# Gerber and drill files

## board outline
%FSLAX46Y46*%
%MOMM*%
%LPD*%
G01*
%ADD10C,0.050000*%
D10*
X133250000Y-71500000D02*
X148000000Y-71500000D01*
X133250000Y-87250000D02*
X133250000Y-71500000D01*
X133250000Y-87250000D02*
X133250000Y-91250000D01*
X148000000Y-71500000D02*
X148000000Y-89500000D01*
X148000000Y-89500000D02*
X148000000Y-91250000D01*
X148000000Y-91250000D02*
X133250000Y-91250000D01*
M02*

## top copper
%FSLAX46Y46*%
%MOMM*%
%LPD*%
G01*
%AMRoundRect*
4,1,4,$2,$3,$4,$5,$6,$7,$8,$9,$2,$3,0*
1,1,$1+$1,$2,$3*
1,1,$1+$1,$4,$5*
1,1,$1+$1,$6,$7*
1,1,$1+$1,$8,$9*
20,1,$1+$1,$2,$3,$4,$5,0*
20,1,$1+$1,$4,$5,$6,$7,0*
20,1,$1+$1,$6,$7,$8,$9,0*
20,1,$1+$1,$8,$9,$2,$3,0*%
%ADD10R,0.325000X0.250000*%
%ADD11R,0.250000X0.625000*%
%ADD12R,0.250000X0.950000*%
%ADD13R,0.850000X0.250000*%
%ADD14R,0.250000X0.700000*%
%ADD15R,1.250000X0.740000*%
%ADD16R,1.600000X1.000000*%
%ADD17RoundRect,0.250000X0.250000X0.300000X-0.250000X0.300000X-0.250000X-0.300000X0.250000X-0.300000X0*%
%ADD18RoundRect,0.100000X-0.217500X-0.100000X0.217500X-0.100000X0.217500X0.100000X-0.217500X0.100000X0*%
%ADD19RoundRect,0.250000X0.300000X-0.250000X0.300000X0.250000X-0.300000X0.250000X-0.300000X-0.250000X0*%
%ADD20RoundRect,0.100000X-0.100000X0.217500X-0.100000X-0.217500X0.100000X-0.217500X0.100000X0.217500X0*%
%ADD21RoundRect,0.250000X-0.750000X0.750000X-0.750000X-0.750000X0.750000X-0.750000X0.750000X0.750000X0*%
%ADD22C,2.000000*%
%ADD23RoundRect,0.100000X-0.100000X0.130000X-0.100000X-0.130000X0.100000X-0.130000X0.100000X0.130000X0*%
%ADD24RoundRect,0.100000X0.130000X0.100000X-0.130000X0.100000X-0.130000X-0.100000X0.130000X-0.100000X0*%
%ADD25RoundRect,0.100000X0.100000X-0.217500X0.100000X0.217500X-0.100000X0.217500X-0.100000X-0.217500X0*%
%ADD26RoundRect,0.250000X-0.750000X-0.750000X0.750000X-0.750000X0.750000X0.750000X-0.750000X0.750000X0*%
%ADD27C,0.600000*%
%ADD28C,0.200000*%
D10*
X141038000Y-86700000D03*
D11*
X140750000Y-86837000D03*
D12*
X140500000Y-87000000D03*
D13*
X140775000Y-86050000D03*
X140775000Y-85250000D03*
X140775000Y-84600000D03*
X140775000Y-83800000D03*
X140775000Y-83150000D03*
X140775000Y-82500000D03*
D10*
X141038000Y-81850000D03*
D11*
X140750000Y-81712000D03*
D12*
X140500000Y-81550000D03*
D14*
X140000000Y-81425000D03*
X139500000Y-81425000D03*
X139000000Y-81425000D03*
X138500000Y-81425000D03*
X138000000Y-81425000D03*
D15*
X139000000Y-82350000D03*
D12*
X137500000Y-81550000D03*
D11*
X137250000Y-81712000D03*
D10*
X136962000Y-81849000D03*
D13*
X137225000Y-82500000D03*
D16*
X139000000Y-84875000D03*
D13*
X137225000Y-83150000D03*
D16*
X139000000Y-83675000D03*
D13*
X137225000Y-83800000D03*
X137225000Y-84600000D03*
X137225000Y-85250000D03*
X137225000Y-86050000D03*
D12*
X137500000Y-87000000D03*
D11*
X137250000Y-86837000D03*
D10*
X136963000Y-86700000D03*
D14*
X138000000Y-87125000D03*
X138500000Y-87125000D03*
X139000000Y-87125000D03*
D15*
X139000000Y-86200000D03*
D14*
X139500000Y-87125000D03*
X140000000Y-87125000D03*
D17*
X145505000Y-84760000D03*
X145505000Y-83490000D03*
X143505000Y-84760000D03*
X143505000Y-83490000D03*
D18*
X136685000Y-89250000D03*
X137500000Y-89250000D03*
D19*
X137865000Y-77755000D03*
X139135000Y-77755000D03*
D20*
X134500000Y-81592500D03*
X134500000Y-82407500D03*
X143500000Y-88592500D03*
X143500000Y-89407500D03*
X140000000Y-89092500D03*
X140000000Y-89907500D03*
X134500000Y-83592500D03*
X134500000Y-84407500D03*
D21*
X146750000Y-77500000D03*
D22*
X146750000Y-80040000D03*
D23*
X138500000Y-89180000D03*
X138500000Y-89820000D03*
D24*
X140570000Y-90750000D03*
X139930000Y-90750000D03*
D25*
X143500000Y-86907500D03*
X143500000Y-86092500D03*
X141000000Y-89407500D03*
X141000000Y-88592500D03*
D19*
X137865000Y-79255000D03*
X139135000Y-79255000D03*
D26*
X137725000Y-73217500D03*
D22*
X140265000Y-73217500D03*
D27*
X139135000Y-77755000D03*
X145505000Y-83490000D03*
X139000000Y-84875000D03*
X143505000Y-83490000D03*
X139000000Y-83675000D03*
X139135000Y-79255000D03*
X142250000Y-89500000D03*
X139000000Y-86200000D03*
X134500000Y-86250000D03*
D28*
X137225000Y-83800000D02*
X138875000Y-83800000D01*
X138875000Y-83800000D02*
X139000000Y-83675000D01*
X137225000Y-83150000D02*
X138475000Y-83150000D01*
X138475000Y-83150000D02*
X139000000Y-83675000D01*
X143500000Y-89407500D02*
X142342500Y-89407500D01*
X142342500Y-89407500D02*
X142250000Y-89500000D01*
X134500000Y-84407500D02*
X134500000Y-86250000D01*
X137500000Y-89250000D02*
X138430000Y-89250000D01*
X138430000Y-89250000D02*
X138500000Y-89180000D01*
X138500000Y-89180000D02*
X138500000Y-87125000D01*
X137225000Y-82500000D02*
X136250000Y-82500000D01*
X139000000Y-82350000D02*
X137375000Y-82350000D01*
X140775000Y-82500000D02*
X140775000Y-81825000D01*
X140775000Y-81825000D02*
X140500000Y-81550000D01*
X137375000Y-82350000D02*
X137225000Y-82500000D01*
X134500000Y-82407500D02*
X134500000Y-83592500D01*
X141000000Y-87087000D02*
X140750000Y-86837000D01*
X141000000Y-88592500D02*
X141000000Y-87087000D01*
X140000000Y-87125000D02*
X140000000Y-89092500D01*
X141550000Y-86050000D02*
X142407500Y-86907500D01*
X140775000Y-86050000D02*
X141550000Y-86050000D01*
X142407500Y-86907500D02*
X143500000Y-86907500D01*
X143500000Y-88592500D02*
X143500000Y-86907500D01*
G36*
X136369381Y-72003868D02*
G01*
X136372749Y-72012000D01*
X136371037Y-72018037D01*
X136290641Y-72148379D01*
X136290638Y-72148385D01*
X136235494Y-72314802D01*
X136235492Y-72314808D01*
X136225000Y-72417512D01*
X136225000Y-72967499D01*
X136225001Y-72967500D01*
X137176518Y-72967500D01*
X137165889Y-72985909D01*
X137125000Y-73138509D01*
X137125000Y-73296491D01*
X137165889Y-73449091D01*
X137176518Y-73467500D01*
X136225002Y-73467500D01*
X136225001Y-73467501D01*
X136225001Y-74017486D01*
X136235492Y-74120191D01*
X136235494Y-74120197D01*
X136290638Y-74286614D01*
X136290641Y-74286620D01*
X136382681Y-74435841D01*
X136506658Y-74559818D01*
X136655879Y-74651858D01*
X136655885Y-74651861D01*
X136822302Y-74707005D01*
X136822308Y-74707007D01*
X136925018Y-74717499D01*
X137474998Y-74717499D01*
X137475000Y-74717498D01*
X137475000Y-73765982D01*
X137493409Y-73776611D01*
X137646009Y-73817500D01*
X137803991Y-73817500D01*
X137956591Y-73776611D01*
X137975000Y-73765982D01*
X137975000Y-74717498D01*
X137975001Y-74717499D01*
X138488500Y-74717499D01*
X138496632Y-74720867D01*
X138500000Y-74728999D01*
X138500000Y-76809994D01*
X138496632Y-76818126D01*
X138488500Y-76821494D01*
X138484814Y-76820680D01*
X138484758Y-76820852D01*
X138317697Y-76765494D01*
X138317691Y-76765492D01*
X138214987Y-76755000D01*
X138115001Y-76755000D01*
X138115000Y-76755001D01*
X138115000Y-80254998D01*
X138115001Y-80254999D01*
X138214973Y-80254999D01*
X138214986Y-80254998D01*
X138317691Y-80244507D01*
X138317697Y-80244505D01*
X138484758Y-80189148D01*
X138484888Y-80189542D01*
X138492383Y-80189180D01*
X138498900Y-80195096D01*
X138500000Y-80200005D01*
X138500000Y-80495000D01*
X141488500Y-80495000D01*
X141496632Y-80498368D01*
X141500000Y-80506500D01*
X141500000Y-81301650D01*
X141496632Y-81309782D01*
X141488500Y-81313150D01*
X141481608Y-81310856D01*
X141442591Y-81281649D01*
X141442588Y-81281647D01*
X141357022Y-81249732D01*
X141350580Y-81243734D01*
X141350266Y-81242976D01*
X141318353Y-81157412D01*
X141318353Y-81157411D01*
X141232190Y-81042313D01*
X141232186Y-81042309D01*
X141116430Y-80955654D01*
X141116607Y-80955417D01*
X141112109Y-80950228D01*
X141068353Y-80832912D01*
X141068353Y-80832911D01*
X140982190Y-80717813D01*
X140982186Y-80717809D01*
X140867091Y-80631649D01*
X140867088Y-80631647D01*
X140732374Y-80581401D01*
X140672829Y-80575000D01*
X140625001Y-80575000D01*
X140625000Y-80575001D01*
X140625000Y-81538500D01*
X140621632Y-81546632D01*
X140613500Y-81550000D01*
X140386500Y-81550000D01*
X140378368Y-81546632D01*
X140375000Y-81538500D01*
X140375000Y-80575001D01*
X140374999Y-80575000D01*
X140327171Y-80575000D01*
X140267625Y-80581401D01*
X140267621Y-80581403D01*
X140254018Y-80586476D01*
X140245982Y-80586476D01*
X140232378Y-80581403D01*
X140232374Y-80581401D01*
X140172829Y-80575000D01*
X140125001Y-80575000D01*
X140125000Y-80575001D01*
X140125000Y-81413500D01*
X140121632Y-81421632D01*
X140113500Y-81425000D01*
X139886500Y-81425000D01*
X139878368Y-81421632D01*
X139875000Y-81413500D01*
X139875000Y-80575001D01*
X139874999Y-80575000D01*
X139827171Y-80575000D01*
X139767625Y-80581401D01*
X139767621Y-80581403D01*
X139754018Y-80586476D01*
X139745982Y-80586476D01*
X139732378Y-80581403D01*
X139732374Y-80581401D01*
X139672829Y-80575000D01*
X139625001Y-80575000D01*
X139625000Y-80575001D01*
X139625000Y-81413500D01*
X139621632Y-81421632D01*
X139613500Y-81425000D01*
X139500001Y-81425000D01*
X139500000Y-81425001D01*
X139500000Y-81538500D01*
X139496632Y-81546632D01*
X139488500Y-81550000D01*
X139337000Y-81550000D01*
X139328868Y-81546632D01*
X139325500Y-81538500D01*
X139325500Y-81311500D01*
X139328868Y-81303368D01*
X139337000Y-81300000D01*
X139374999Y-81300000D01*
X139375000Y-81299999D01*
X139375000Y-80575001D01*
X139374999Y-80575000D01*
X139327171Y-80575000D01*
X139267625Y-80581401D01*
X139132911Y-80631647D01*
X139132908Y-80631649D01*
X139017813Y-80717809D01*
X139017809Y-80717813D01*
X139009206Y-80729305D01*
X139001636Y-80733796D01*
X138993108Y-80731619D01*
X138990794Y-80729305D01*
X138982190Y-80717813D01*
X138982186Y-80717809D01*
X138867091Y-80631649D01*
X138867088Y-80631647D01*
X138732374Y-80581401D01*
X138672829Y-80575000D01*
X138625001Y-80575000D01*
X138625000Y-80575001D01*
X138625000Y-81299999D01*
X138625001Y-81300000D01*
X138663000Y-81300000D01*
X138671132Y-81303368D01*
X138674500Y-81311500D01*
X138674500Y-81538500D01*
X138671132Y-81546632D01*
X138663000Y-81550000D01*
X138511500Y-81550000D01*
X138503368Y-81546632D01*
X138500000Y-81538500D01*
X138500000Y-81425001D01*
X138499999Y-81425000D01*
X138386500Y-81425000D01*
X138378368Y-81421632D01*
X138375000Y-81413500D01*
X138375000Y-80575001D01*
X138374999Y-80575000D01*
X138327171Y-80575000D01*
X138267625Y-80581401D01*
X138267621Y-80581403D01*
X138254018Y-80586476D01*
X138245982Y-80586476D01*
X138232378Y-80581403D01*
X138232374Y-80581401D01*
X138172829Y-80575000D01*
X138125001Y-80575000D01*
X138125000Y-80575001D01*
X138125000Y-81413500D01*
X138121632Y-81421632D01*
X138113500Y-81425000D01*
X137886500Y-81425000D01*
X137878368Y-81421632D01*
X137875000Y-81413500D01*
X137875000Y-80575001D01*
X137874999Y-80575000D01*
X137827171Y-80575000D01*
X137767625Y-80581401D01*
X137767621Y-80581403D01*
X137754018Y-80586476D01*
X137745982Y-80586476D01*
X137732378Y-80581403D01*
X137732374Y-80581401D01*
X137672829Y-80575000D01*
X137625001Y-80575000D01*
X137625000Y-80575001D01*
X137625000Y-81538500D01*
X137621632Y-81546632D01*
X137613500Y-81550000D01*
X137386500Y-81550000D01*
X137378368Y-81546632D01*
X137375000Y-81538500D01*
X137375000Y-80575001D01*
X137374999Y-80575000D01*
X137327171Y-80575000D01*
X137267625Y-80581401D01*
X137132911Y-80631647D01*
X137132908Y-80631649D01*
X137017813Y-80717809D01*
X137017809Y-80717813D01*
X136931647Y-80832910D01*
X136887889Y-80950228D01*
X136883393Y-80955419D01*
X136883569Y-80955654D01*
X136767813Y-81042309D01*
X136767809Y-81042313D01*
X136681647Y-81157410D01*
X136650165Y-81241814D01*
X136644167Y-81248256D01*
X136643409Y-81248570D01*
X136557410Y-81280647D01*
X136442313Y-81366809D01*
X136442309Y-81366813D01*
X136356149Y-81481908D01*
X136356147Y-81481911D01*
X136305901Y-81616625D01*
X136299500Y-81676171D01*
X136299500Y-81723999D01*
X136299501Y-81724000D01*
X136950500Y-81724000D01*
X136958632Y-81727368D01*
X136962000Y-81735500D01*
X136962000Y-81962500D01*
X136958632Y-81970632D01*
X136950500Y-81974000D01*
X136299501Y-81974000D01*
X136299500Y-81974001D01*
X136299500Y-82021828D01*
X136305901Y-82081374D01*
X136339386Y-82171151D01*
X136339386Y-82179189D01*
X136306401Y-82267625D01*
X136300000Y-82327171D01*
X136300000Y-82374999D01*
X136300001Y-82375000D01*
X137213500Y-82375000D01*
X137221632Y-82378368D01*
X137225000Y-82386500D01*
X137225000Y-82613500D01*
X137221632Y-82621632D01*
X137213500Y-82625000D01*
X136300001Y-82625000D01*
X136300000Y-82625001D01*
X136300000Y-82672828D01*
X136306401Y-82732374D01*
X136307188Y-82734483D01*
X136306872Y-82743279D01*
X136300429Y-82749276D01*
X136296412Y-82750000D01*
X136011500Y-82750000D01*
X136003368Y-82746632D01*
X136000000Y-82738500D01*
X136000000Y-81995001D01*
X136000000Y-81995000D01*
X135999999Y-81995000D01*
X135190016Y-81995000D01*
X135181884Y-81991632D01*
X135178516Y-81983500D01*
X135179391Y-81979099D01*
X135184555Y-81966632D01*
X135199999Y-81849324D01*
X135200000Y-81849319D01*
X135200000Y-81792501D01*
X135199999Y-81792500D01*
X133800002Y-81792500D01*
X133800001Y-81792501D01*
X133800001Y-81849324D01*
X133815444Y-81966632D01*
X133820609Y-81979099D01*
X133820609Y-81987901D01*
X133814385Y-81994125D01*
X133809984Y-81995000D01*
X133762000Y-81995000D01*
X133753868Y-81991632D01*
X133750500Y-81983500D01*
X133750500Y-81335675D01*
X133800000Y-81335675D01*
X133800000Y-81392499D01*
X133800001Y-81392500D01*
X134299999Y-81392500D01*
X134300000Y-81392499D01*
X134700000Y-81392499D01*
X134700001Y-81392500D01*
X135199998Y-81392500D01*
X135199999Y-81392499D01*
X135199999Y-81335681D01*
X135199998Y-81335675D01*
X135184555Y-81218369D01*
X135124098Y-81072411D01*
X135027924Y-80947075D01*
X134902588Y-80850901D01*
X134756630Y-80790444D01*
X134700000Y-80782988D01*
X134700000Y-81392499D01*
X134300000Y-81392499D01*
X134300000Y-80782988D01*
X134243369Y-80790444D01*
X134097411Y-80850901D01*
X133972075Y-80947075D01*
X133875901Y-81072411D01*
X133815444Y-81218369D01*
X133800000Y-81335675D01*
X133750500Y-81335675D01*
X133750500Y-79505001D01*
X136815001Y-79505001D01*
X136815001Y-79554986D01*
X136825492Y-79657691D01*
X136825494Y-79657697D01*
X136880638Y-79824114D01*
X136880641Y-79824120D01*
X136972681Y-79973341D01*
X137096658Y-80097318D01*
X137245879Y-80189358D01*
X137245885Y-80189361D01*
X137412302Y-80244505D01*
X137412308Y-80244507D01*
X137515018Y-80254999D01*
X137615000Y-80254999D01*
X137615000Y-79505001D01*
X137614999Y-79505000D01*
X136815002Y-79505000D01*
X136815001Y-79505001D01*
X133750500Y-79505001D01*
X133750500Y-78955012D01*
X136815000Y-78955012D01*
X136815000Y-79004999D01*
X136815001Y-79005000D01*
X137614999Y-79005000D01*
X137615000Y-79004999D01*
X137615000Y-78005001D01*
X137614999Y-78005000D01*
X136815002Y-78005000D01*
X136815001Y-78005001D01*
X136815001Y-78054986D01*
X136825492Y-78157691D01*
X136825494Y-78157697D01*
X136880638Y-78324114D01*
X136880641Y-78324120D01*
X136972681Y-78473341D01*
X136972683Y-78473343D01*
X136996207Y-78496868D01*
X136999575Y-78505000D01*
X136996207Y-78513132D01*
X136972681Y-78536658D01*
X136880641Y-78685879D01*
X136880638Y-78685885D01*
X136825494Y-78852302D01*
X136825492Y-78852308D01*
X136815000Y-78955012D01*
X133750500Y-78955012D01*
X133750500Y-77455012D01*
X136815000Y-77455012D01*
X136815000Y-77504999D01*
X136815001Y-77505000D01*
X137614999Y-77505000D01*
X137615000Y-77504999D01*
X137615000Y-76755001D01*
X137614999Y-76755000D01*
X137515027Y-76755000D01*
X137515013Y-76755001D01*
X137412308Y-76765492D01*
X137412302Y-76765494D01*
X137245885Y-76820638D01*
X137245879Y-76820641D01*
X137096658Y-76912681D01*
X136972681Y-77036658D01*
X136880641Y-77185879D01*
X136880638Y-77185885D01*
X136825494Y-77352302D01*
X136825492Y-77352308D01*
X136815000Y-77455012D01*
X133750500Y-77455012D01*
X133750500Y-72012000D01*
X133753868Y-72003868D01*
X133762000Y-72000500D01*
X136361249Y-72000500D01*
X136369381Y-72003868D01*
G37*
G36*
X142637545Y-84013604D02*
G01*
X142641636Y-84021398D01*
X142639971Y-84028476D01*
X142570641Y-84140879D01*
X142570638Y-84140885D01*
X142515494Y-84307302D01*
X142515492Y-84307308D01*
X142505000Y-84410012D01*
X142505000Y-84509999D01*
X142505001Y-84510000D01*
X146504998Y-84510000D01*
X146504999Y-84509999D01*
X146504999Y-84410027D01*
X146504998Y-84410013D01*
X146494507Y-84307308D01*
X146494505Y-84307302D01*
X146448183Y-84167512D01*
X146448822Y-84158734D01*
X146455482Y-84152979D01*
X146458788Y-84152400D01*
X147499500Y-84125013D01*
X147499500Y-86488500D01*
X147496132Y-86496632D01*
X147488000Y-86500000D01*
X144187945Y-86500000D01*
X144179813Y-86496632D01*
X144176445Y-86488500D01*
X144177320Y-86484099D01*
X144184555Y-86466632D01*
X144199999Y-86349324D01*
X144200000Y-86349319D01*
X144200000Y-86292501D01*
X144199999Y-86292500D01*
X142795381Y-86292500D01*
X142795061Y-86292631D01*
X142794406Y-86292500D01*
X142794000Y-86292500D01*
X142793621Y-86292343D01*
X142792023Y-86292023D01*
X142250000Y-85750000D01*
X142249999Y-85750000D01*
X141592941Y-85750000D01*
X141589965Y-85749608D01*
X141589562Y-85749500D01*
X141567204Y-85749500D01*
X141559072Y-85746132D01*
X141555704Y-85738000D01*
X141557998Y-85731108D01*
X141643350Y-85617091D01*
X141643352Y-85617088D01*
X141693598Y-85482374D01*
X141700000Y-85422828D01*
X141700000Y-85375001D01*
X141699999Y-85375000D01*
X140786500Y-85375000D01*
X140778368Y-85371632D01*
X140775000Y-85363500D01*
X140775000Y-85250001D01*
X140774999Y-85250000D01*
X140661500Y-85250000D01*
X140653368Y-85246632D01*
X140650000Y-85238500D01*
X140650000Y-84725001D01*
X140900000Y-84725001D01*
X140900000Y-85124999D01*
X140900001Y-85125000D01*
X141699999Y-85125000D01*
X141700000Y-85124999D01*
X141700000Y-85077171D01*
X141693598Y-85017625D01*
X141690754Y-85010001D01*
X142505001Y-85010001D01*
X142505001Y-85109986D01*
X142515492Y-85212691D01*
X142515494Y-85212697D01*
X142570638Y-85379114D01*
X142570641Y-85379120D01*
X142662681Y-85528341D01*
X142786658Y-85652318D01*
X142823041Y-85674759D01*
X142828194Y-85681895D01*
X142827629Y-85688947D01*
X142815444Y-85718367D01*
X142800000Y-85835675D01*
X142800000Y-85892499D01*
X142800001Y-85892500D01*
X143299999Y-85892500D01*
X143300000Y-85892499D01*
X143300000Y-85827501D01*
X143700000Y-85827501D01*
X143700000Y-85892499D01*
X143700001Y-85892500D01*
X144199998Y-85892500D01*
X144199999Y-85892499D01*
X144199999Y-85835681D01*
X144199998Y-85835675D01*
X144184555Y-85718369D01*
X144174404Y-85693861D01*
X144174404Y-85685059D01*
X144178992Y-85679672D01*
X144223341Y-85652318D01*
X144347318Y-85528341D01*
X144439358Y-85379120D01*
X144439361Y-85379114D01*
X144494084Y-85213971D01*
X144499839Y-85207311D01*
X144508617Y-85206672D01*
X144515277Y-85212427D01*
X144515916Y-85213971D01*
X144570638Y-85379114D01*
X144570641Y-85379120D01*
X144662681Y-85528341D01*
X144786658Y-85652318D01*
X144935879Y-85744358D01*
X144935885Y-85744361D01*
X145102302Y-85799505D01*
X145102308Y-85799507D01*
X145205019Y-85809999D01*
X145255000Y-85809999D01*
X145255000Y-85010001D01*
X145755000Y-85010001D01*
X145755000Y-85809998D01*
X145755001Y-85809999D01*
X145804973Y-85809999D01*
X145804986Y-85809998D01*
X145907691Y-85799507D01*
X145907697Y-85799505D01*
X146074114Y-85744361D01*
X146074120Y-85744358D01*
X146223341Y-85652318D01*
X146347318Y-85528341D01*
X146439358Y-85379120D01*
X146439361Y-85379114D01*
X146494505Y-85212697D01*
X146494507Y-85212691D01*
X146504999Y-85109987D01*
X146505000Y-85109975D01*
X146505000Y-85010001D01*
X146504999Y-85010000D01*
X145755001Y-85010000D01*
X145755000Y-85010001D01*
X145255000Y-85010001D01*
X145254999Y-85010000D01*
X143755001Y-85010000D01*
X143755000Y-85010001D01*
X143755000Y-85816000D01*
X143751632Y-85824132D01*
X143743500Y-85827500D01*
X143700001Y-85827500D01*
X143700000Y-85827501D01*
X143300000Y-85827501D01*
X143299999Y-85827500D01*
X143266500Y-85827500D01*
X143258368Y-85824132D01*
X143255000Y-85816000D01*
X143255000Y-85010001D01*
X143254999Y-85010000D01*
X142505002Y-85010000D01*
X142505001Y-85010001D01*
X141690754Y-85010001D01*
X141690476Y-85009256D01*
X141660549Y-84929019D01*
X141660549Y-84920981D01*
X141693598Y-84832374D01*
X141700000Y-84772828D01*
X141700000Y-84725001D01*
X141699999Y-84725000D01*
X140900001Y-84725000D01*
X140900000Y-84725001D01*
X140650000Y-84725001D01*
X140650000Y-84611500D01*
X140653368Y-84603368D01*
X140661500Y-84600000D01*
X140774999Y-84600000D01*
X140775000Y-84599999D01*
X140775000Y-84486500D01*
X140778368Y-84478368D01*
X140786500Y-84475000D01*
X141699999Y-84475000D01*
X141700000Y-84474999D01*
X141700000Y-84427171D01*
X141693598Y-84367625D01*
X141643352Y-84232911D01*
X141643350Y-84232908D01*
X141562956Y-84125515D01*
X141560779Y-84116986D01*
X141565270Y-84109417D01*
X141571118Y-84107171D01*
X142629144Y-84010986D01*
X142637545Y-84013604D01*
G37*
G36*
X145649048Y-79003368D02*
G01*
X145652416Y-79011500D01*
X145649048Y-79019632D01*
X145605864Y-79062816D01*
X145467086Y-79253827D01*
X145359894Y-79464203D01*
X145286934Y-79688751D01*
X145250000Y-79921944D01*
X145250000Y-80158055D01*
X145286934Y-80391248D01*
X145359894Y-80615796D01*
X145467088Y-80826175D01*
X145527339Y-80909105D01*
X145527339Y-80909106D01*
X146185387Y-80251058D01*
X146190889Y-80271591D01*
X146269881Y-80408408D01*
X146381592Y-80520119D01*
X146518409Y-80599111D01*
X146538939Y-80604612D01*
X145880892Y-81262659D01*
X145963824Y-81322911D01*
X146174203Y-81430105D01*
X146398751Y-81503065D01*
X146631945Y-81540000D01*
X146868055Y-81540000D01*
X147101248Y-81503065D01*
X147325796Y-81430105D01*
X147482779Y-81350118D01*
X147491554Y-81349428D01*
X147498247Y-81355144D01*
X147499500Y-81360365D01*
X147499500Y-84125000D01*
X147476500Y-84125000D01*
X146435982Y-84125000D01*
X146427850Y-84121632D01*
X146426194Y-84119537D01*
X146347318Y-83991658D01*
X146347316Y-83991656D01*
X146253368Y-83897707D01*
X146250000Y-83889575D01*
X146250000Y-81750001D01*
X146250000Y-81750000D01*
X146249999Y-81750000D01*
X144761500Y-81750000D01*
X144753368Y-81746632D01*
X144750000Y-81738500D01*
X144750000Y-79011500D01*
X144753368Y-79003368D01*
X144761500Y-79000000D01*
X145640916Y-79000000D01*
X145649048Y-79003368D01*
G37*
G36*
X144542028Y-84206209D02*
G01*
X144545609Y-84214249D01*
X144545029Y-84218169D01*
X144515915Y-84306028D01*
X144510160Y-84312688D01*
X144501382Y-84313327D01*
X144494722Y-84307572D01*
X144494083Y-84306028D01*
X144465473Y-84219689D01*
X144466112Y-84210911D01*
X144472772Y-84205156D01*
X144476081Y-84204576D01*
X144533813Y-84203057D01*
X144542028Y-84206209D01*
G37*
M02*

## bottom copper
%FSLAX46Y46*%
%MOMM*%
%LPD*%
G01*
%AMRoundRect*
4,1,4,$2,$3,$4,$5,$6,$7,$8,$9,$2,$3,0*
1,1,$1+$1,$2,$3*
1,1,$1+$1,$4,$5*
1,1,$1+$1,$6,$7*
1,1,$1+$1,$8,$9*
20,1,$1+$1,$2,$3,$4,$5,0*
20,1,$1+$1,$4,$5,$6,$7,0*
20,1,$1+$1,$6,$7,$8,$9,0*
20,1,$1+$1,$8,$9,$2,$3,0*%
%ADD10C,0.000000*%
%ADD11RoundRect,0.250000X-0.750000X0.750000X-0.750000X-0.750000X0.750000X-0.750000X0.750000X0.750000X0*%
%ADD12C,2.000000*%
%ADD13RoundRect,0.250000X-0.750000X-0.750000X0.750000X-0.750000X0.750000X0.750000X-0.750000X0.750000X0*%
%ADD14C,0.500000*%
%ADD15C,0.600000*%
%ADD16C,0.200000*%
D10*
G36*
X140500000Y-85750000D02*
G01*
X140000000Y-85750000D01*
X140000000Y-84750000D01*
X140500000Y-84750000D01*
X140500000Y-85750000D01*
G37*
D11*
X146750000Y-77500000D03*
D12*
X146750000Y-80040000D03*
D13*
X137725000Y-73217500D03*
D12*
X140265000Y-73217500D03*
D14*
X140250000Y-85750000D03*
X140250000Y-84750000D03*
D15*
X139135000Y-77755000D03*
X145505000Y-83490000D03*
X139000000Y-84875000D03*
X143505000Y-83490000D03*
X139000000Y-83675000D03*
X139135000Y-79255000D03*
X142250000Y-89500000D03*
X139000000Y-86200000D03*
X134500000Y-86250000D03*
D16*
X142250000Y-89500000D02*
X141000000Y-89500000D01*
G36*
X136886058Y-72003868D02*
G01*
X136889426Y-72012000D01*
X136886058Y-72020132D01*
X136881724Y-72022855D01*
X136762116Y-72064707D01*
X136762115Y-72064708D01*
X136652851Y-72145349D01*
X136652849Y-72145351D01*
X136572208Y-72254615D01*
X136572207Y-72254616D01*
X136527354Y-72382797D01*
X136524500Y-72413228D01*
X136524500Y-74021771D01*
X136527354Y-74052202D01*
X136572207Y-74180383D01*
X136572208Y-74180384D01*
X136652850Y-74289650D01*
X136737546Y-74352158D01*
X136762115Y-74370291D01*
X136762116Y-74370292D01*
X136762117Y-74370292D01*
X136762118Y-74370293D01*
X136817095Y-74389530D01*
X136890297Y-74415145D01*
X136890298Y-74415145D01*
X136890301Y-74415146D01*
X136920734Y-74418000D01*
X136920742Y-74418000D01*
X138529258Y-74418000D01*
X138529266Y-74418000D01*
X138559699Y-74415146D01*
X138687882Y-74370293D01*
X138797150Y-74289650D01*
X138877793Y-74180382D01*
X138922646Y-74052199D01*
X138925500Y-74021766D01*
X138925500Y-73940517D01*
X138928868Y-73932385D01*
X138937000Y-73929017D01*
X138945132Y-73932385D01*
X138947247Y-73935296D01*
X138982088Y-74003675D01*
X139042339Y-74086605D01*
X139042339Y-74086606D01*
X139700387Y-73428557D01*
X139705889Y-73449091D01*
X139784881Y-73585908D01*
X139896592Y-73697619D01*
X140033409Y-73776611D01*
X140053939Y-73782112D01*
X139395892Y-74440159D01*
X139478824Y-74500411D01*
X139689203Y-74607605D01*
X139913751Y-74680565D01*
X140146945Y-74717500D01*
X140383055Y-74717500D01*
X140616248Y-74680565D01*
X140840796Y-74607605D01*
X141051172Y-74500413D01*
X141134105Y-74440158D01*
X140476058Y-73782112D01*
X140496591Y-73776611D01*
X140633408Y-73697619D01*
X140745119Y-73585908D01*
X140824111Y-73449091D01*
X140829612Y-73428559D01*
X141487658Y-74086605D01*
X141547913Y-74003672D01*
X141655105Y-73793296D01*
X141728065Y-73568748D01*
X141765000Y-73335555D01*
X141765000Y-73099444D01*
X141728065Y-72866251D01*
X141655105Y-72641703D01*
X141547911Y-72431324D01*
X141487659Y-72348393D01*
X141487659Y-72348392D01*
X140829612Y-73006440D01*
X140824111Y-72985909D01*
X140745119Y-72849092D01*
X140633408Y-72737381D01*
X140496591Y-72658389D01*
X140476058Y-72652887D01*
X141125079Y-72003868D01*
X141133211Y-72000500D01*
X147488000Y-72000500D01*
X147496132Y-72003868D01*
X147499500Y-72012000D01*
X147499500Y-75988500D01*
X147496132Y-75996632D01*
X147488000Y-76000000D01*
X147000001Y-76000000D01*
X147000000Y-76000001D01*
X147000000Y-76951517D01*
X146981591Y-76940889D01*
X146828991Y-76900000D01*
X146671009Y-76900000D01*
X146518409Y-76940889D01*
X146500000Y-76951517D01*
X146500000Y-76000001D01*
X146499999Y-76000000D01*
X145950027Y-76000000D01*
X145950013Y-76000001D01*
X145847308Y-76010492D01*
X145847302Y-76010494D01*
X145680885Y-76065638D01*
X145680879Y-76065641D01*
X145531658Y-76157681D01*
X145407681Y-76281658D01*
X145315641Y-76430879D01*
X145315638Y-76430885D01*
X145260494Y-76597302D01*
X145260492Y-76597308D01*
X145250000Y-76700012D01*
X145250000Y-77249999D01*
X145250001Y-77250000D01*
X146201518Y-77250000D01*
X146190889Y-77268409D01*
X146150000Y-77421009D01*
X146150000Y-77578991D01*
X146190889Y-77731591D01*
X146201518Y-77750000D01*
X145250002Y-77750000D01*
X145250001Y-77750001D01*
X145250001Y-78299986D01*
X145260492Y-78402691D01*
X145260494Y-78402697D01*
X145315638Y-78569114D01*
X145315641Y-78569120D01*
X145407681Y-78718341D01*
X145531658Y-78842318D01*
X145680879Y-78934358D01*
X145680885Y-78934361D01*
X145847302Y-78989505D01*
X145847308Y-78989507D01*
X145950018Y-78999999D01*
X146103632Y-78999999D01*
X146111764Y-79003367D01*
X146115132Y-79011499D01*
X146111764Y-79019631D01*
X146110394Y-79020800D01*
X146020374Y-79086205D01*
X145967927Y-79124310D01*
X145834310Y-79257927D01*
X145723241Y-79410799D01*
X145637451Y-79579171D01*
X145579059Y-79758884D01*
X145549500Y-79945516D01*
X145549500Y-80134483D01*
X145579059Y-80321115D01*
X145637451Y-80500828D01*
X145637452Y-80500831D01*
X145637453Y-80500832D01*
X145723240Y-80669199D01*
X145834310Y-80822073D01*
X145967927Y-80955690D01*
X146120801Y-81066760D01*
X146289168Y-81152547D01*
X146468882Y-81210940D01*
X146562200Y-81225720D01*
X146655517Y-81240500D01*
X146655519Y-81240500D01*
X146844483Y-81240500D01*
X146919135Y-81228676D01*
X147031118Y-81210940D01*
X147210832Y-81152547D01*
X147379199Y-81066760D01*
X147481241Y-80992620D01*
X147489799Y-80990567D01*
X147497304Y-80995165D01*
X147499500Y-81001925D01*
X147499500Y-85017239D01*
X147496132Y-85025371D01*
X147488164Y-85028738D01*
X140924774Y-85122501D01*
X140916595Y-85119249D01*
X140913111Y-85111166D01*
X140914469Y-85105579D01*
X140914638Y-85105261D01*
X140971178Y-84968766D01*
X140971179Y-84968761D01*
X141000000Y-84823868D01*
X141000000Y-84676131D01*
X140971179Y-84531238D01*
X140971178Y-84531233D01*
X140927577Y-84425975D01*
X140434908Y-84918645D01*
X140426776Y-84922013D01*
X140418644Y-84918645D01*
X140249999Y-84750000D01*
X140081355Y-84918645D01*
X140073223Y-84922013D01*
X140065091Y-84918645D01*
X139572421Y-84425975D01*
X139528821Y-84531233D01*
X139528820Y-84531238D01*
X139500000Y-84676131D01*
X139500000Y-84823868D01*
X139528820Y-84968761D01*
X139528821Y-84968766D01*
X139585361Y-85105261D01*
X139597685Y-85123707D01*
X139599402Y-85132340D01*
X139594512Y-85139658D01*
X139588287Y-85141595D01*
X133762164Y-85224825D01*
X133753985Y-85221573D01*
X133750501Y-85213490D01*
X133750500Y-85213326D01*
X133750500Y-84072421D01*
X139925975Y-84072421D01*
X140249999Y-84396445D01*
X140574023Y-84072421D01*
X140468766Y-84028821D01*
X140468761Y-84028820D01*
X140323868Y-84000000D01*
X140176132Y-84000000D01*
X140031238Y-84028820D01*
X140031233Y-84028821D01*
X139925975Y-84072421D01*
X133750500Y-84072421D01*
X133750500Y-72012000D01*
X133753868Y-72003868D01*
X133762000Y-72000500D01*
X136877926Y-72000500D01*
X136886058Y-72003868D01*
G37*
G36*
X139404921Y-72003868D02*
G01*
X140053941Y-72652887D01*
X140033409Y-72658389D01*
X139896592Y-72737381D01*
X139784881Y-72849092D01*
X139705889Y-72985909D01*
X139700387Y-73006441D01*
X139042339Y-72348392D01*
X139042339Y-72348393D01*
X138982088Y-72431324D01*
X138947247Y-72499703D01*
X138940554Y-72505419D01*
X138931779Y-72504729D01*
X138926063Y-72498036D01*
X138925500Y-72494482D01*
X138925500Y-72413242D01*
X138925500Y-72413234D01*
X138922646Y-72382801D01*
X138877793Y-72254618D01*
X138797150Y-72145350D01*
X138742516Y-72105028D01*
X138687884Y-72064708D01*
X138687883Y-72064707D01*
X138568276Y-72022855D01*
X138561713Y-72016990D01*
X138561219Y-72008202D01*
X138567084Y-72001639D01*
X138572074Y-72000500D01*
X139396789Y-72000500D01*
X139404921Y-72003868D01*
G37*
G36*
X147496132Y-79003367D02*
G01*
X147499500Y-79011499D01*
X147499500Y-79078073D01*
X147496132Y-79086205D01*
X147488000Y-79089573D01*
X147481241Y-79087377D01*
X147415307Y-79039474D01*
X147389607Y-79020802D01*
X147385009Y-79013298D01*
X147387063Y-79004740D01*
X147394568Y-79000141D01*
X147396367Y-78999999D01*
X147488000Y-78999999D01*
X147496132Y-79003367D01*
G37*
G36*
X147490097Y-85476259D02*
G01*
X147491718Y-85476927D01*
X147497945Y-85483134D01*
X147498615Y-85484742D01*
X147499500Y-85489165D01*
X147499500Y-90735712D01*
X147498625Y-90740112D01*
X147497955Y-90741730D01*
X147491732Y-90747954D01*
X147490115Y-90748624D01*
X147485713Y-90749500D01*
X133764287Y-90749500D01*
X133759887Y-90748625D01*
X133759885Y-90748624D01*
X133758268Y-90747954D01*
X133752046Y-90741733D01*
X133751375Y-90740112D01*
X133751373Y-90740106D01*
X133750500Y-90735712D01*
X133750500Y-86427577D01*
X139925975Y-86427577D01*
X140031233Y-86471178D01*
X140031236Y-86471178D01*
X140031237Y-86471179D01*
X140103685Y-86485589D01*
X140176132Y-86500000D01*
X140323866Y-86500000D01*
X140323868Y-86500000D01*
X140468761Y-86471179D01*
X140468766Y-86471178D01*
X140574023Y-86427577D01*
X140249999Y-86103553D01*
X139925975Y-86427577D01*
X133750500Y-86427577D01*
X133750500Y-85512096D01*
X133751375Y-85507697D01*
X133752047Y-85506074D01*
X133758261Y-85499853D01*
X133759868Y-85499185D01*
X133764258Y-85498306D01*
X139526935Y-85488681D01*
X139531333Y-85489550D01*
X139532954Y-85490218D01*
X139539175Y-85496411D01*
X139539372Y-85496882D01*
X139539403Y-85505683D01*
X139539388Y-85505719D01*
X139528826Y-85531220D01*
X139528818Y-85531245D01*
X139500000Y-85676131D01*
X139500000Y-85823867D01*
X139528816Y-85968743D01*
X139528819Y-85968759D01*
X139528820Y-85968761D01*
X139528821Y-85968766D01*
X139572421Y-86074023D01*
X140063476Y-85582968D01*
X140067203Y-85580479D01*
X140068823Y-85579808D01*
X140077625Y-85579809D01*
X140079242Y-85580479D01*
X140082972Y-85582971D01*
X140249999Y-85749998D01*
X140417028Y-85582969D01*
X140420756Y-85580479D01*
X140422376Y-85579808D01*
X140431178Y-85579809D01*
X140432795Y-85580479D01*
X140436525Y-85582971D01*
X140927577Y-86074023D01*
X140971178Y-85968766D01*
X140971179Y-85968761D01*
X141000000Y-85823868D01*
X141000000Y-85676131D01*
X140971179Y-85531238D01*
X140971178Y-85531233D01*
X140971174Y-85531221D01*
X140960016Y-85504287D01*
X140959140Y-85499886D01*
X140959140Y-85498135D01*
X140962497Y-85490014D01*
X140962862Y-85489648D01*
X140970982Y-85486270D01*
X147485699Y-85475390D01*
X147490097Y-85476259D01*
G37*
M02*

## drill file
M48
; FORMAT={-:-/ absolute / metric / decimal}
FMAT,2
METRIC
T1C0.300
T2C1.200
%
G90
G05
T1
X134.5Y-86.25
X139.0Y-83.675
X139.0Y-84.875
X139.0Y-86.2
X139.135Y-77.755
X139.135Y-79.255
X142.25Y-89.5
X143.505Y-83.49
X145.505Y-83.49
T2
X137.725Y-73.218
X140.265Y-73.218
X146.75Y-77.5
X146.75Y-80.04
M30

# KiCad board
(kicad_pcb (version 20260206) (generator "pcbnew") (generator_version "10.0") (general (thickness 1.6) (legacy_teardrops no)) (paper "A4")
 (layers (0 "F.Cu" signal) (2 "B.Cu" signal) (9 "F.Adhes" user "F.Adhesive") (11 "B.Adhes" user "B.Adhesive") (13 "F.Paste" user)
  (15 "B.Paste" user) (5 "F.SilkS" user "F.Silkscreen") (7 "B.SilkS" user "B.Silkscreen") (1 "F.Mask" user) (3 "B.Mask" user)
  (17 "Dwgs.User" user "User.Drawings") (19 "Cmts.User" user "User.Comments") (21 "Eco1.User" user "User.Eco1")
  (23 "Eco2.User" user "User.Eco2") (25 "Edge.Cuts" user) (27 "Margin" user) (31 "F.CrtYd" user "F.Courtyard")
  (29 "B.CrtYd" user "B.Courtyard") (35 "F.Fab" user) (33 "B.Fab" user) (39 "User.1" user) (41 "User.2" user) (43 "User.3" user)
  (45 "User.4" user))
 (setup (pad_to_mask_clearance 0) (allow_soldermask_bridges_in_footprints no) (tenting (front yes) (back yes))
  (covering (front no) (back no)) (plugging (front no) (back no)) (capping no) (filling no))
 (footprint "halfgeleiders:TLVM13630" (layer "F.Cu") (at 139 84.275 180)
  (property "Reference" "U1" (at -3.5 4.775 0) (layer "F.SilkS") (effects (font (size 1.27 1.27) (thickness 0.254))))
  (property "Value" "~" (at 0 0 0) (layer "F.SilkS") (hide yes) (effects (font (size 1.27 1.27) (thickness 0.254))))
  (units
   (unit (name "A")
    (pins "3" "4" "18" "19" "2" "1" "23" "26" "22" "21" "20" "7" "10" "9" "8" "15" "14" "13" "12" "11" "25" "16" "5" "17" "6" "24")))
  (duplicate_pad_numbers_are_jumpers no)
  (pad "1" smd rect (at -2.038 -2.425 270) (size 0.25 0.325) (layers "F.Cu" "F.Mask" "F.Paste") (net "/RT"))
  (pad "1" smd rect (at -1.75 -2.562 180) (size 0.25 0.625) (layers "F.Cu" "F.Mask" "F.Paste") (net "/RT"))
  (pad "1" smd rect (at -1.5 -2.725 180) (size 0.25 0.95) (layers "F.Cu" "F.Mask" "F.Paste") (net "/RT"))
  (pad "2" smd rect (at -1.775 -1.775 270) (size 0.25 0.85) (layers "F.Cu" "F.Mask" "F.Paste") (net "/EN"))
  (pad "3" smd rect (at -1.775 -0.975 270) (size 0.25 0.85) (layers "F.Cu" "F.Mask" "F.Paste") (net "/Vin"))
  (pad "4" smd rect (at -1.775 -0.325 270) (size 0.25 0.85) (layers "F.Cu" "F.Mask" "F.Paste") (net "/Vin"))
  (pad "5" smd rect (at -1.775 0.475 270) (size 0.25 0.85) (layers "F.Cu" "F.Mask" "F.Paste") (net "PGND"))
  (pad "6" smd rect (at -1.775 1.125 270) (size 0.25 0.85) (layers "F.Cu" "F.Mask" "F.Paste") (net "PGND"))
  (pad "7" smd rect (at -1.775 1.775 270) (size 0.25 0.85) (layers "F.Cu" "F.Mask" "F.Paste") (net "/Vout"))
  (pad "8" smd rect (at -2.038 2.425 270) (size 0.25 0.325) (layers "F.Cu" "F.Mask" "F.Paste") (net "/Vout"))
  (pad "8" smd rect (at -1.75 2.563 180) (size 0.25 0.625) (layers "F.Cu" "F.Mask" "F.Paste") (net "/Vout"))
  (pad "8" smd rect (at -1.5 2.725 180) (size 0.25 0.95) (layers "F.Cu" "F.Mask" "F.Paste") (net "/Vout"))
  (pad "9" smd rect (at -1 2.85 180) (size 0.25 0.7) (layers "F.Cu" "F.Mask" "F.Paste") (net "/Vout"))
  (pad "10" smd rect (at -0.5 2.85 180) (size 0.25 0.7) (layers "F.Cu" "F.Mask" "F.Paste") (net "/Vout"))
  (pad "11" smd rect (at 0 2.85 180) (size 0.25 0.7) (layers "F.Cu" "F.Mask" "F.Paste") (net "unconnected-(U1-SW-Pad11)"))
  (pad "12" smd rect (at 0.5 2.85 180) (size 0.25 0.7) (layers "F.Cu" "F.Mask" "F.Paste") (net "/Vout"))
  (pad "13" smd rect (at 1 2.85 180) (size 0.25 0.7) (layers "F.Cu" "F.Mask" "F.Paste") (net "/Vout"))
  (pad "14" smd rect (at 0 1.925 270) (size 0.74 1.25) (layers "F.Cu" "F.Mask" "F.Paste") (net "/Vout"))
  (pad "14" smd rect (at 1.5 2.725 180) (size 0.25 0.95) (layers "F.Cu" "F.Mask" "F.Paste") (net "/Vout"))
  (pad "14" smd rect (at 1.75 2.563 180) (size 0.25 0.625) (layers "F.Cu" "F.Mask" "F.Paste") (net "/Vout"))
  (pad "14" smd rect (at 2.038 2.426 270) (size 0.25 0.325) (layers "F.Cu" "F.Mask" "F.Paste") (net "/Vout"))
  (pad "15" smd rect (at 1.775 1.775 270) (size 0.25 0.85) (layers "F.Cu" "F.Mask" "F.Paste") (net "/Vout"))
  (pad "16" smd rect (at 0 -0.6 270) (size 1 1.6) (layers "F.Cu" "F.Mask" "F.Paste") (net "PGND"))
  (pad "16" smd rect (at 1.775 1.125 270) (size 0.25 0.85) (layers "F.Cu" "F.Mask" "F.Paste") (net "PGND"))
  (pad "17" smd rect (at 0 0.6 270) (size 1 1.6) (layers "F.Cu" "F.Mask" "F.Paste") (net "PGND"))
  (pad "17" smd rect (at 1.775 0.475 270) (size 0.25 0.85) (layers "F.Cu" "F.Mask" "F.Paste") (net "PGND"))
  (pad "18" smd rect (at 1.775 -0.325 270) (size 0.25 0.85) (layers "F.Cu" "F.Mask" "F.Paste") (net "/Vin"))
  (pad "19" smd rect (at 1.775 -0.975 270) (size 0.25 0.85) (layers "F.Cu" "F.Mask" "F.Paste") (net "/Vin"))
  (pad "20" smd rect (at 1.775 -1.775 270) (size 0.25 0.85) (layers "F.Cu" "F.Mask" "F.Paste") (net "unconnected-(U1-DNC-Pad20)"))
  (pad "21" smd rect (at 1.5 -2.725 180) (size 0.25 0.95) (layers "F.Cu" "F.Mask" "F.Paste") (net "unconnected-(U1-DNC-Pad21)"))
  (pad "21" smd rect (at 1.75 -2.562 180) (size 0.25 0.625) (layers "F.Cu" "F.Mask" "F.Paste") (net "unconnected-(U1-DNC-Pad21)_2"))
  (pad "21" smd rect (at 2.037 -2.425 270) (size 0.25 0.325) (layers "F.Cu" "F.Mask" "F.Paste") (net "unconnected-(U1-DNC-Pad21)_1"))
  (pad "22" smd rect (at 1 -2.85 180) (size 0.25 0.7) (layers "F.Cu" "F.Mask" "F.Paste") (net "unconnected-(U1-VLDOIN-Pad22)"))
  (pad "23" smd rect (at 0.5 -2.85 180) (size 0.25 0.7) (layers "F.Cu" "F.Mask" "F.Paste") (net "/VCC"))
  (pad "24" smd rect (at 0 -2.85 180) (size 0.25 0.7) (layers "F.Cu" "F.Mask" "F.Paste") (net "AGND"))
  (pad "24" smd rect (at 0 -1.925 270) (size 0.74 1.25) (layers "F.Cu" "F.Mask" "F.Paste") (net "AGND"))
  (pad "25" smd rect (at -0.5 -2.85 180) (size 0.25 0.7) (layers "F.Cu" "F.Mask" "F.Paste") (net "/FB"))
  (pad "26" smd rect (at -1 -2.85 180) (size 0.25 0.7) (layers "F.Cu" "F.Mask" "F.Paste") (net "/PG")))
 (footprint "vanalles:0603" (layer "F.Cu") (at 145.5 84.125 90)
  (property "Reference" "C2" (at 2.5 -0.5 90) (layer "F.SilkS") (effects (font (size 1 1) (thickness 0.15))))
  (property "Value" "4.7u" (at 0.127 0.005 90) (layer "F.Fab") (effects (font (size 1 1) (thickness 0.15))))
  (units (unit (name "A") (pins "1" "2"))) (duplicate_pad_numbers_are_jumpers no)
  (pad "1" smd roundrect (at -0.635 0.005 180) (size 1 1.1) (layers "F.Cu" "F.Mask" "F.Paste") (roundrect_rratio 0.25) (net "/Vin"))
  (pad "2" smd roundrect (at 0.635 0.005 180) (size 1 1.1) (layers "F.Cu" "F.Mask" "F.Paste") (roundrect_rratio 0.25) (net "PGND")))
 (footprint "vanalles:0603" (layer "F.Cu") (at 143.5 84.125 90)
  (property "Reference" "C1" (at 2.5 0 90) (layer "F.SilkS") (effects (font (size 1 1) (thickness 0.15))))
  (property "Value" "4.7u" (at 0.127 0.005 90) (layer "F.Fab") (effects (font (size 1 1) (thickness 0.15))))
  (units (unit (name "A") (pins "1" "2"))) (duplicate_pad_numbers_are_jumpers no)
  (pad "1" smd roundrect (at -0.635 0.005 180) (size 1 1.1) (layers "F.Cu" "F.Mask" "F.Paste") (roundrect_rratio 0.25) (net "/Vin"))
  (pad "2" smd roundrect (at 0.635 0.005 180) (size 1 1.1) (layers "F.Cu" "F.Mask" "F.Paste") (roundrect_rratio 0.25) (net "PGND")))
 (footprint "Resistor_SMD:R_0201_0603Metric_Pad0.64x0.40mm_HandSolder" (layer "F.Cu") (at 137.0925 89.25)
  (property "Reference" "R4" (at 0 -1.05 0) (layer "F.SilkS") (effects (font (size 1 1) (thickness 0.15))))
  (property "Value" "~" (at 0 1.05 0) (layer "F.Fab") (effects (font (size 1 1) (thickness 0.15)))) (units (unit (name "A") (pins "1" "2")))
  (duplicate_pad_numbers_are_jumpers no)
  (pad "" smd roundrect (at -0.4325 0) (size 0.458 0.36) (layers "F.Paste") (roundrect_rratio 0.25))
  (pad "" smd roundrect (at 0.4325 0) (size 0.458 0.36) (layers "F.Paste") (roundrect_rratio 0.25))
  (pad "1" smd roundrect (at -0.4075 0) (size 0.635 0.4) (layers "F.Cu" "F.Mask") (roundrect_rratio 0.25) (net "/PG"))
  (pad "2" smd roundrect (at 0.4075 0) (size 0.635 0.4) (layers "F.Cu" "F.Mask") (roundrect_rratio 0.25) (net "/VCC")))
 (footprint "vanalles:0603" (layer "F.Cu") (at 138.5 77.75)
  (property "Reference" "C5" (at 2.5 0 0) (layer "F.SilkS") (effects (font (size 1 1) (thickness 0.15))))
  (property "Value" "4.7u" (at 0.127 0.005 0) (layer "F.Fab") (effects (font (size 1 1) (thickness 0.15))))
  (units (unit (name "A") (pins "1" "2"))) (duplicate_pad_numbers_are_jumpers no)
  (pad "1" smd roundrect (at -0.635 0.005 90) (size 1 1.1) (layers "F.Cu" "F.Mask" "F.Paste") (roundrect_rratio 0.25) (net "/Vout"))
  (pad "2" smd roundrect (at 0.635 0.005 90) (size 1 1.1) (layers "F.Cu" "F.Mask" "F.Paste") (roundrect_rratio 0.25) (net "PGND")))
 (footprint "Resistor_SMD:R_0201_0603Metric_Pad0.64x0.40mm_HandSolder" (layer "F.Cu") (at 134.5 82 -90)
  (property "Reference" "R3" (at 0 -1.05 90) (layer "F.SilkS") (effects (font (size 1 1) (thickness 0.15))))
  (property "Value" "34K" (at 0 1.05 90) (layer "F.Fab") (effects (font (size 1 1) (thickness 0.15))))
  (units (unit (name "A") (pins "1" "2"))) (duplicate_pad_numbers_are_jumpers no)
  (pad "" smd roundrect (at -0.4325 0 270) (size 0.458 0.36) (layers "F.Paste") (roundrect_rratio 0.25))
  (pad "" smd roundrect (at 0.4325 0 270) (size 0.458 0.36) (layers "F.Paste") (roundrect_rratio 0.25))
  (pad "1" smd roundrect (at -0.4075 0 270) (size 0.635 0.4) (layers "F.Cu" "F.Mask") (roundrect_rratio 0.25) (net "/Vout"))
  (pad "2" smd roundrect (at 0.4075 0 270) (size 0.635 0.4) (layers "F.Cu" "F.Mask") (roundrect_rratio 0.25) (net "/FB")))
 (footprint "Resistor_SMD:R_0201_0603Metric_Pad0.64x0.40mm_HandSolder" (layer "F.Cu") (at 143.5 89 -90)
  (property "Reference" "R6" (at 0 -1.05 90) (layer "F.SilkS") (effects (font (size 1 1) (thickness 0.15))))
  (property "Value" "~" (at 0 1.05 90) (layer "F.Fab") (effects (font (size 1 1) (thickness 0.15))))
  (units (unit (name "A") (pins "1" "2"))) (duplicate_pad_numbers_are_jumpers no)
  (pad "" smd roundrect (at -0.4325 0 270) (size 0.458 0.36) (layers "F.Paste") (roundrect_rratio 0.25))
  (pad "" smd roundrect (at 0.4325 0 270) (size 0.458 0.36) (layers "F.Paste") (roundrect_rratio 0.25))
  (pad "1" smd roundrect (at -0.4075 0 270) (size 0.635 0.4) (layers "F.Cu" "F.Mask") (roundrect_rratio 0.25) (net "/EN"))
  (pad "2" smd roundrect (at 0.4075 0 270) (size 0.635 0.4) (layers "F.Cu" "F.Mask") (roundrect_rratio 0.25) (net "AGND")))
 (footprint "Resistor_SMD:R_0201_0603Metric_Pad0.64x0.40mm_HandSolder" (layer "F.Cu") (at 140 89.5 -90)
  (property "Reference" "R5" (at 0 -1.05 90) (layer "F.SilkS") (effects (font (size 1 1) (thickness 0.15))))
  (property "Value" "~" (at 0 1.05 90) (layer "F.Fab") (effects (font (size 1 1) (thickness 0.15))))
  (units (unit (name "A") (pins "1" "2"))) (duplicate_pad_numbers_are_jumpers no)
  (pad "" smd roundrect (at -0.4325 0 270) (size 0.458 0.36) (layers "F.Paste") (roundrect_rratio 0.25))
  (pad "" smd roundrect (at 0.4325 0 270) (size 0.458 0.36) (layers "F.Paste") (roundrect_rratio 0.25))
  (pad "1" smd roundrect (at -0.4075 0 270) (size 0.635 0.4) (layers "F.Cu" "F.Mask") (roundrect_rratio 0.25) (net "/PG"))
  (pad "2" smd roundrect (at 0.4075 0 270) (size 0.635 0.4) (layers "F.Cu" "F.Mask") (roundrect_rratio 0.25) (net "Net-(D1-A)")))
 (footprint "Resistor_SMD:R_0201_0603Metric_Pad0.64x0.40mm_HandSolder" (layer "F.Cu") (at 134.5 84 -90)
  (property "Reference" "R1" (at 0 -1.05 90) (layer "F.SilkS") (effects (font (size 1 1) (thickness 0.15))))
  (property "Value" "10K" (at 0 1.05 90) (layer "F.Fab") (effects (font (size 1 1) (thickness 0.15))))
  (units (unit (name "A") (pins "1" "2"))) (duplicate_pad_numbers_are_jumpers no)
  (pad "" smd roundrect (at -0.4325 0 270) (size 0.458 0.36) (layers "F.Paste") (roundrect_rratio 0.25))
  (pad "" smd roundrect (at 0.4325 0 270) (size 0.458 0.36) (layers "F.Paste") (roundrect_rratio 0.25))
  (pad "1" smd roundrect (at -0.4075 0 270) (size 0.635 0.4) (layers "F.Cu" "F.Mask") (roundrect_rratio 0.25) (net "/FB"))
  (pad "2" smd roundrect (at 0.4075 0 270) (size 0.635 0.4) (layers "F.Cu" "F.Mask") (roundrect_rratio 0.25) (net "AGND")))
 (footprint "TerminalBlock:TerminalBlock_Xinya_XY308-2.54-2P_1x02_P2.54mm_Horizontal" (layer "F.Cu") (at 146.75 77.5 -90)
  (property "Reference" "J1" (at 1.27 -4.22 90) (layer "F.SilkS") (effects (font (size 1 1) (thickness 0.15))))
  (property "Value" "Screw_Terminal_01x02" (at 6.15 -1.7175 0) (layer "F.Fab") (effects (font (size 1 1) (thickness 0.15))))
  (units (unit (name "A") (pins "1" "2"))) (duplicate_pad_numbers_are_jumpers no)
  (pad "1" thru_hole roundrect (at 0 0 270) (size 2 2) (drill 1.2) (layers "*.Cu" "*.Mask") (remove_unused_layers no)
   (roundrect_rratio 0.125) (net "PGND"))
  (pad "2" thru_hole circle (at 2.54 0 270) (size 2 2) (drill 1.2) (layers "*.Cu" "*.Mask") (remove_unused_layers no) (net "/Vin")))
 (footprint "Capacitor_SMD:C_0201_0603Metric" (layer "F.Cu") (at 138.5 89.5 -90)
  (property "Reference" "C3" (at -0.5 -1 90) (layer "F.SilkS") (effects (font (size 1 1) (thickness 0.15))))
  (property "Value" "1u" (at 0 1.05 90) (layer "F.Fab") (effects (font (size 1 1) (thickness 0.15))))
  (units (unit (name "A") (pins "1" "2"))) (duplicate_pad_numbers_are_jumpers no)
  (pad "" smd roundrect (at -0.345 0 270) (size 0.318 0.36) (layers "F.Paste") (roundrect_rratio 0.25))
  (pad "" smd roundrect (at 0.345 0 270) (size 0.318 0.36) (layers "F.Paste") (roundrect_rratio 0.25))
  (pad "1" smd roundrect (at -0.32 0 270) (size 0.46 0.4) (layers "F.Cu" "F.Mask") (roundrect_rratio 0.25) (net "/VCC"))
  (pad "2" smd roundrect (at 0.32 0 270) (size 0.46 0.4) (layers "F.Cu" "F.Mask") (roundrect_rratio 0.25) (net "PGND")))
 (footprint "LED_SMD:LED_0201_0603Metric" (layer "F.Cu") (at 140.25 90.75 180)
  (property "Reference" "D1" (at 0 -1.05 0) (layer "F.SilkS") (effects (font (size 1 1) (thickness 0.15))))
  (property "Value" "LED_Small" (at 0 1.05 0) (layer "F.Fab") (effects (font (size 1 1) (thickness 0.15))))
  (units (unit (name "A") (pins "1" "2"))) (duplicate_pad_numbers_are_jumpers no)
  (pad "" smd roundrect (at -0.345 0 180) (size 0.318 0.36) (layers "F.Paste") (roundrect_rratio 0.25))
  (pad "" smd roundrect (at 0.345 0 180) (size 0.318 0.36) (layers "F.Paste") (roundrect_rratio 0.25))
  (pad "1" smd roundrect (at -0.32 0 180) (size 0.46 0.4) (layers "F.Cu" "F.Mask") (roundrect_rratio 0.25) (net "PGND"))
  (pad "2" smd roundrect (at 0.32 0 180) (size 0.46 0.4) (layers "F.Cu" "F.Mask") (roundrect_rratio 0.25) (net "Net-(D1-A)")))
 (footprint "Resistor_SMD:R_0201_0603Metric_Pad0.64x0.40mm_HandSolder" (layer "F.Cu") (at 143.5 86.5 90)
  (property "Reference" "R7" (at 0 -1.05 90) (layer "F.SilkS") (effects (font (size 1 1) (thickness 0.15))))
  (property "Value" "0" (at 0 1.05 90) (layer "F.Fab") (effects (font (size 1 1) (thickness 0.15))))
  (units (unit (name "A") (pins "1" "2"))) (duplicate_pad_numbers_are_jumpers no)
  (pad "" smd roundrect (at -0.4325 0 90) (size 0.458 0.36) (layers "F.Paste") (roundrect_rratio 0.25))
  (pad "" smd roundrect (at 0.4325 0 90) (size 0.458 0.36) (layers "F.Paste") (roundrect_rratio 0.25))
  (pad "1" smd roundrect (at -0.4075 0 90) (size 0.635 0.4) (layers "F.Cu" "F.Mask") (roundrect_rratio 0.25) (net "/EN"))
  (pad "2" smd roundrect (at 0.4075 0 90) (size 0.635 0.4) (layers "F.Cu" "F.Mask") (roundrect_rratio 0.25) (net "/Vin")))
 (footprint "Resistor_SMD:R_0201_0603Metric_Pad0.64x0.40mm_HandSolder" (layer "F.Cu") (at 141 89 90)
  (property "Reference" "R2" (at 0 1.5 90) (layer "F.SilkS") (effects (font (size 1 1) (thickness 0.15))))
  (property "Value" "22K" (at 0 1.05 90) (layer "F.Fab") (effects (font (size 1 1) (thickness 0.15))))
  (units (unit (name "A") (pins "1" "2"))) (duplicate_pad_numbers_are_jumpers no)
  (pad "" smd roundrect (at -0.4325 0 90) (size 0.458 0.36) (layers "F.Paste") (roundrect_rratio 0.25))
  (pad "" smd roundrect (at 0.4325 0 90) (size 0.458 0.36) (layers "F.Paste") (roundrect_rratio 0.25))
  (pad "1" smd roundrect (at -0.4075 0 90) (size 0.635 0.4) (layers "F.Cu" "F.Mask") (roundrect_rratio 0.25) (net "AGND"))
  (pad "2" smd roundrect (at 0.4075 0 90) (size 0.635 0.4) (layers "F.Cu" "F.Mask") (roundrect_rratio 0.25) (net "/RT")))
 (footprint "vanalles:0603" (layer "F.Cu") (at 138.5 79.25)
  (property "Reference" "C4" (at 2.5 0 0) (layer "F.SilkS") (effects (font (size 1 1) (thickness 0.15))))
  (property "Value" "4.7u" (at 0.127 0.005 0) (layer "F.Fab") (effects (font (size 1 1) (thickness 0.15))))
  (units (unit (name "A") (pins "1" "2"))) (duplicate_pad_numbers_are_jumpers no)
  (pad "1" smd roundrect (at -0.635 0.005 90) (size 1 1.1) (layers "F.Cu" "F.Mask" "F.Paste") (roundrect_rratio 0.25) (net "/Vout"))
  (pad "2" smd roundrect (at 0.635 0.005 90) (size 1 1.1) (layers "F.Cu" "F.Mask" "F.Paste") (roundrect_rratio 0.25) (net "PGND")))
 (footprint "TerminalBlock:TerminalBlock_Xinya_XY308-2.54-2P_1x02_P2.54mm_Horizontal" (layer "F.Cu") (at 137.725 73.2175)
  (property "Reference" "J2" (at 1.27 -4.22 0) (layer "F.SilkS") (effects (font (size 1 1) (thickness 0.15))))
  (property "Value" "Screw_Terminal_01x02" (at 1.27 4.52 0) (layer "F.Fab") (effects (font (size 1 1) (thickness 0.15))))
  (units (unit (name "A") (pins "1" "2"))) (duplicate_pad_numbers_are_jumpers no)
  (pad "1" thru_hole roundrect (at 0 0) (size 2 2) (drill 1.2) (layers "*.Cu" "*.Mask") (remove_unused_layers no) (roundrect_rratio 0.125)
   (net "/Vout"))
  (pad "2" thru_hole circle (at 2.54 0) (size 2 2) (drill 1.2) (layers "*.Cu" "*.Mask") (remove_unused_layers no) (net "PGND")))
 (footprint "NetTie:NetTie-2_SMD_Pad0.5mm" (layer "B.Cu") (at 140.25 85.25 90)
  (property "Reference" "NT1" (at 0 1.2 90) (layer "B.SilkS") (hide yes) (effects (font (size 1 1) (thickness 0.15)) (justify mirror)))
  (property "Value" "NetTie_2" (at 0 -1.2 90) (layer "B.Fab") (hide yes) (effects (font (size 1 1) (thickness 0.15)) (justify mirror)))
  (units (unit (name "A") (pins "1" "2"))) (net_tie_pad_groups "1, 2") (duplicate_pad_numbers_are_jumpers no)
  (fp_poly (pts (xy -0.5 0.25) (xy 0.5 0.25) (xy 0.5 -0.25) (xy -0.5 -0.25)) (stroke (width 0) (type solid)) (fill yes) (layer "B.Cu"))
  (pad "1" smd circle (at -0.5 0 90) (size 0.5 0.5) (layers "B.Cu") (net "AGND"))
  (pad "2" smd circle (at 0.5 0 90) (size 0.5 0.5) (layers "B.Cu") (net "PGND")))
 (gr_line (start 133.25 71.5) (end 148 71.5) (stroke (width 0.05) (type default)) (layer "Edge.Cuts"))
 (gr_line (start 133.25 87.25) (end 133.25 71.5) (stroke (width 0.05) (type default)) (layer "Edge.Cuts"))
 (gr_line (start 133.25 87.25) (end 133.25 91.25) (stroke (width 0.05) (type default)) (layer "Edge.Cuts"))
 (gr_line (start 148 71.5) (end 148 89.5) (stroke (width 0.05) (type default)) (layer "Edge.Cuts"))
 (gr_line (start 148 89.5) (end 148 91.25) (stroke (width 0.05) (type default)) (layer "Edge.Cuts"))
 (gr_line (start 148 91.25) (end 133.25 91.25) (stroke (width 0.05) (type default)) (layer "Edge.Cuts"))
 (segment (start 137.225 83.8) (end 138.875 83.8) (width 0.2) (layer "F.Cu") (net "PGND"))
 (segment (start 138.875 83.8) (end 139 83.675) (width 0.2) (layer "F.Cu") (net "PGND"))
 (segment (start 137.225 83.15) (end 138.475 83.15) (width 0.2) (layer "F.Cu") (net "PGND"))
 (segment (start 138.475 83.15) (end 139 83.675) (width 0.2) (layer "F.Cu") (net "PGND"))
 (via (at 139.135 77.755) (size 0.6) (drill 0.3) (layers "F.Cu" "B.Cu") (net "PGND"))
 (via (at 145.505 83.49) (size 0.6) (drill 0.3) (layers "F.Cu" "B.Cu") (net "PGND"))
 (via (at 139 84.875) (size 0.6) (drill 0.3) (layers "F.Cu" "B.Cu") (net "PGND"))
 (via (at 143.505 83.49) (size 0.6) (drill 0.3) (layers "F.Cu" "B.Cu") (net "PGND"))
 (via (at 139 83.675) (size 0.6) (drill 0.3) (layers "F.Cu" "B.Cu") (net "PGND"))
 (via (at 139.135 79.255) (size 0.6) (drill 0.3) (layers "F.Cu" "B.Cu") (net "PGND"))
 (segment (start 143.5 89.4075) (end 142.3425 89.4075) (width 0.2) (layer "F.Cu") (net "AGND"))
 (segment (start 142.3425 89.4075) (end 142.25 89.5) (width 0.2) (layer "F.Cu") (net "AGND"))
 (segment (start 134.5 84.4075) (end 134.5 86.25) (width 0.2) (layer "F.Cu") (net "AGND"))
 (via (at 142.25 89.5) (size 0.6) (drill 0.3) (layers "F.Cu" "B.Cu") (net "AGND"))
 (via (at 139 86.2) (size 0.6) (drill 0.3) (layers "F.Cu" "B.Cu") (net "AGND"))
 (via (at 134.5 86.25) (size 0.6) (drill 0.3) (layers "F.Cu" "B.Cu") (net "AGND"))
 (segment (start 142.25 89.5) (end 141 89.5) (width 0.2) (layer "B.Cu") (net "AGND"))
 (segment (start 137.5 89.25) (end 138.43 89.25) (width 0.2) (layer "F.Cu") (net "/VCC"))
 (segment (start 138.43 89.25) (end 138.5 89.18) (width 0.2) (layer "F.Cu") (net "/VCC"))
 (segment (start 138.5 89.18) (end 138.5 87.125) (width 0.2) (layer "F.Cu") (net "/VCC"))
 (segment (start 137.225 82.5) (end 136.25 82.5) (width 0.2) (layer "F.Cu") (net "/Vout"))
 (segment (start 139 82.35) (end 137.375 82.35) (width 0.2) (layer "F.Cu") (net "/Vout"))
 (segment (start 140.775 82.5) (end 140.775 81.825) (width 0.2) (layer "F.Cu") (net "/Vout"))
 (segment (start 140.775 81.825) (end 140.5 81.55) (width 0.2) (layer "F.Cu") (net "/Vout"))
 (segment (start 137.375 82.35) (end 137.225 82.5) (width 0.2) (layer "F.Cu") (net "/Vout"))
 (segment (start 134.5 82.4075) (end 134.5 83.5925) (width 0.2) (layer "F.Cu") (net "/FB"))
 (segment (start 141 87.087) (end 140.75 86.837) (width 0.2) (layer "F.Cu") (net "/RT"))
 (segment (start 141 88.5925) (end 141 87.087) (width 0.2) (layer "F.Cu") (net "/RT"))
 (segment (start 140 87.125) (end 140 89.0925) (width 0.2) (layer "F.Cu") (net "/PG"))
 (segment (start 141.55 86.05) (end 142.4075 86.9075) (width 0.2) (layer "F.Cu") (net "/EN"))
 (segment (start 140.775 86.05) (end 141.55 86.05) (width 0.2) (layer "F.Cu") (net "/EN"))
 (segment (start 142.4075 86.9075) (end 143.5 86.9075) (width 0.2) (layer "F.Cu") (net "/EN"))
 (segment (start 143.5 88.5925) (end 143.5 86.9075) (width 0.2) (layer "F.Cu") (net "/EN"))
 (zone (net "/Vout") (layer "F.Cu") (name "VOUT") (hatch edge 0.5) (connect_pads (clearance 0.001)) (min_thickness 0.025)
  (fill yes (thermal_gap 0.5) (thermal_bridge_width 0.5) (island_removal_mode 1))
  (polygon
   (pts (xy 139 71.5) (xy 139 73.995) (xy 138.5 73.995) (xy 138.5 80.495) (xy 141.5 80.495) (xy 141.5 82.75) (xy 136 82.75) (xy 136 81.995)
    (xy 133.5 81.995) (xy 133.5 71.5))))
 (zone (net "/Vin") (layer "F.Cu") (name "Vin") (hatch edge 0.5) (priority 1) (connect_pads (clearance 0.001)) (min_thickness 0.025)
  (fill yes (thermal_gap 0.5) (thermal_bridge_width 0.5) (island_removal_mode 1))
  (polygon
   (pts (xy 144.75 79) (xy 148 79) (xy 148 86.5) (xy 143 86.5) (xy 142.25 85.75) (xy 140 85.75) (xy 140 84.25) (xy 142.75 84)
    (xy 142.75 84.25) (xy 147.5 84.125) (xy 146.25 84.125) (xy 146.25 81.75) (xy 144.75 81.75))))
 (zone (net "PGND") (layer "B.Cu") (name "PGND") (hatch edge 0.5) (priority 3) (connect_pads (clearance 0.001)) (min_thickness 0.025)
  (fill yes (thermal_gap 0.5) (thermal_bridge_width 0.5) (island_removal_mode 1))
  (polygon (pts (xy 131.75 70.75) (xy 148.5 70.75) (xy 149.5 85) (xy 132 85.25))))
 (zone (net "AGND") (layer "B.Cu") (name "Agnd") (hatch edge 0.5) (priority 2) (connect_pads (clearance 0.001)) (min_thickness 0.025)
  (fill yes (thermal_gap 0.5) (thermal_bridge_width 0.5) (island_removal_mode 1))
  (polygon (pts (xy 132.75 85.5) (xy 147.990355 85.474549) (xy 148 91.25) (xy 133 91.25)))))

